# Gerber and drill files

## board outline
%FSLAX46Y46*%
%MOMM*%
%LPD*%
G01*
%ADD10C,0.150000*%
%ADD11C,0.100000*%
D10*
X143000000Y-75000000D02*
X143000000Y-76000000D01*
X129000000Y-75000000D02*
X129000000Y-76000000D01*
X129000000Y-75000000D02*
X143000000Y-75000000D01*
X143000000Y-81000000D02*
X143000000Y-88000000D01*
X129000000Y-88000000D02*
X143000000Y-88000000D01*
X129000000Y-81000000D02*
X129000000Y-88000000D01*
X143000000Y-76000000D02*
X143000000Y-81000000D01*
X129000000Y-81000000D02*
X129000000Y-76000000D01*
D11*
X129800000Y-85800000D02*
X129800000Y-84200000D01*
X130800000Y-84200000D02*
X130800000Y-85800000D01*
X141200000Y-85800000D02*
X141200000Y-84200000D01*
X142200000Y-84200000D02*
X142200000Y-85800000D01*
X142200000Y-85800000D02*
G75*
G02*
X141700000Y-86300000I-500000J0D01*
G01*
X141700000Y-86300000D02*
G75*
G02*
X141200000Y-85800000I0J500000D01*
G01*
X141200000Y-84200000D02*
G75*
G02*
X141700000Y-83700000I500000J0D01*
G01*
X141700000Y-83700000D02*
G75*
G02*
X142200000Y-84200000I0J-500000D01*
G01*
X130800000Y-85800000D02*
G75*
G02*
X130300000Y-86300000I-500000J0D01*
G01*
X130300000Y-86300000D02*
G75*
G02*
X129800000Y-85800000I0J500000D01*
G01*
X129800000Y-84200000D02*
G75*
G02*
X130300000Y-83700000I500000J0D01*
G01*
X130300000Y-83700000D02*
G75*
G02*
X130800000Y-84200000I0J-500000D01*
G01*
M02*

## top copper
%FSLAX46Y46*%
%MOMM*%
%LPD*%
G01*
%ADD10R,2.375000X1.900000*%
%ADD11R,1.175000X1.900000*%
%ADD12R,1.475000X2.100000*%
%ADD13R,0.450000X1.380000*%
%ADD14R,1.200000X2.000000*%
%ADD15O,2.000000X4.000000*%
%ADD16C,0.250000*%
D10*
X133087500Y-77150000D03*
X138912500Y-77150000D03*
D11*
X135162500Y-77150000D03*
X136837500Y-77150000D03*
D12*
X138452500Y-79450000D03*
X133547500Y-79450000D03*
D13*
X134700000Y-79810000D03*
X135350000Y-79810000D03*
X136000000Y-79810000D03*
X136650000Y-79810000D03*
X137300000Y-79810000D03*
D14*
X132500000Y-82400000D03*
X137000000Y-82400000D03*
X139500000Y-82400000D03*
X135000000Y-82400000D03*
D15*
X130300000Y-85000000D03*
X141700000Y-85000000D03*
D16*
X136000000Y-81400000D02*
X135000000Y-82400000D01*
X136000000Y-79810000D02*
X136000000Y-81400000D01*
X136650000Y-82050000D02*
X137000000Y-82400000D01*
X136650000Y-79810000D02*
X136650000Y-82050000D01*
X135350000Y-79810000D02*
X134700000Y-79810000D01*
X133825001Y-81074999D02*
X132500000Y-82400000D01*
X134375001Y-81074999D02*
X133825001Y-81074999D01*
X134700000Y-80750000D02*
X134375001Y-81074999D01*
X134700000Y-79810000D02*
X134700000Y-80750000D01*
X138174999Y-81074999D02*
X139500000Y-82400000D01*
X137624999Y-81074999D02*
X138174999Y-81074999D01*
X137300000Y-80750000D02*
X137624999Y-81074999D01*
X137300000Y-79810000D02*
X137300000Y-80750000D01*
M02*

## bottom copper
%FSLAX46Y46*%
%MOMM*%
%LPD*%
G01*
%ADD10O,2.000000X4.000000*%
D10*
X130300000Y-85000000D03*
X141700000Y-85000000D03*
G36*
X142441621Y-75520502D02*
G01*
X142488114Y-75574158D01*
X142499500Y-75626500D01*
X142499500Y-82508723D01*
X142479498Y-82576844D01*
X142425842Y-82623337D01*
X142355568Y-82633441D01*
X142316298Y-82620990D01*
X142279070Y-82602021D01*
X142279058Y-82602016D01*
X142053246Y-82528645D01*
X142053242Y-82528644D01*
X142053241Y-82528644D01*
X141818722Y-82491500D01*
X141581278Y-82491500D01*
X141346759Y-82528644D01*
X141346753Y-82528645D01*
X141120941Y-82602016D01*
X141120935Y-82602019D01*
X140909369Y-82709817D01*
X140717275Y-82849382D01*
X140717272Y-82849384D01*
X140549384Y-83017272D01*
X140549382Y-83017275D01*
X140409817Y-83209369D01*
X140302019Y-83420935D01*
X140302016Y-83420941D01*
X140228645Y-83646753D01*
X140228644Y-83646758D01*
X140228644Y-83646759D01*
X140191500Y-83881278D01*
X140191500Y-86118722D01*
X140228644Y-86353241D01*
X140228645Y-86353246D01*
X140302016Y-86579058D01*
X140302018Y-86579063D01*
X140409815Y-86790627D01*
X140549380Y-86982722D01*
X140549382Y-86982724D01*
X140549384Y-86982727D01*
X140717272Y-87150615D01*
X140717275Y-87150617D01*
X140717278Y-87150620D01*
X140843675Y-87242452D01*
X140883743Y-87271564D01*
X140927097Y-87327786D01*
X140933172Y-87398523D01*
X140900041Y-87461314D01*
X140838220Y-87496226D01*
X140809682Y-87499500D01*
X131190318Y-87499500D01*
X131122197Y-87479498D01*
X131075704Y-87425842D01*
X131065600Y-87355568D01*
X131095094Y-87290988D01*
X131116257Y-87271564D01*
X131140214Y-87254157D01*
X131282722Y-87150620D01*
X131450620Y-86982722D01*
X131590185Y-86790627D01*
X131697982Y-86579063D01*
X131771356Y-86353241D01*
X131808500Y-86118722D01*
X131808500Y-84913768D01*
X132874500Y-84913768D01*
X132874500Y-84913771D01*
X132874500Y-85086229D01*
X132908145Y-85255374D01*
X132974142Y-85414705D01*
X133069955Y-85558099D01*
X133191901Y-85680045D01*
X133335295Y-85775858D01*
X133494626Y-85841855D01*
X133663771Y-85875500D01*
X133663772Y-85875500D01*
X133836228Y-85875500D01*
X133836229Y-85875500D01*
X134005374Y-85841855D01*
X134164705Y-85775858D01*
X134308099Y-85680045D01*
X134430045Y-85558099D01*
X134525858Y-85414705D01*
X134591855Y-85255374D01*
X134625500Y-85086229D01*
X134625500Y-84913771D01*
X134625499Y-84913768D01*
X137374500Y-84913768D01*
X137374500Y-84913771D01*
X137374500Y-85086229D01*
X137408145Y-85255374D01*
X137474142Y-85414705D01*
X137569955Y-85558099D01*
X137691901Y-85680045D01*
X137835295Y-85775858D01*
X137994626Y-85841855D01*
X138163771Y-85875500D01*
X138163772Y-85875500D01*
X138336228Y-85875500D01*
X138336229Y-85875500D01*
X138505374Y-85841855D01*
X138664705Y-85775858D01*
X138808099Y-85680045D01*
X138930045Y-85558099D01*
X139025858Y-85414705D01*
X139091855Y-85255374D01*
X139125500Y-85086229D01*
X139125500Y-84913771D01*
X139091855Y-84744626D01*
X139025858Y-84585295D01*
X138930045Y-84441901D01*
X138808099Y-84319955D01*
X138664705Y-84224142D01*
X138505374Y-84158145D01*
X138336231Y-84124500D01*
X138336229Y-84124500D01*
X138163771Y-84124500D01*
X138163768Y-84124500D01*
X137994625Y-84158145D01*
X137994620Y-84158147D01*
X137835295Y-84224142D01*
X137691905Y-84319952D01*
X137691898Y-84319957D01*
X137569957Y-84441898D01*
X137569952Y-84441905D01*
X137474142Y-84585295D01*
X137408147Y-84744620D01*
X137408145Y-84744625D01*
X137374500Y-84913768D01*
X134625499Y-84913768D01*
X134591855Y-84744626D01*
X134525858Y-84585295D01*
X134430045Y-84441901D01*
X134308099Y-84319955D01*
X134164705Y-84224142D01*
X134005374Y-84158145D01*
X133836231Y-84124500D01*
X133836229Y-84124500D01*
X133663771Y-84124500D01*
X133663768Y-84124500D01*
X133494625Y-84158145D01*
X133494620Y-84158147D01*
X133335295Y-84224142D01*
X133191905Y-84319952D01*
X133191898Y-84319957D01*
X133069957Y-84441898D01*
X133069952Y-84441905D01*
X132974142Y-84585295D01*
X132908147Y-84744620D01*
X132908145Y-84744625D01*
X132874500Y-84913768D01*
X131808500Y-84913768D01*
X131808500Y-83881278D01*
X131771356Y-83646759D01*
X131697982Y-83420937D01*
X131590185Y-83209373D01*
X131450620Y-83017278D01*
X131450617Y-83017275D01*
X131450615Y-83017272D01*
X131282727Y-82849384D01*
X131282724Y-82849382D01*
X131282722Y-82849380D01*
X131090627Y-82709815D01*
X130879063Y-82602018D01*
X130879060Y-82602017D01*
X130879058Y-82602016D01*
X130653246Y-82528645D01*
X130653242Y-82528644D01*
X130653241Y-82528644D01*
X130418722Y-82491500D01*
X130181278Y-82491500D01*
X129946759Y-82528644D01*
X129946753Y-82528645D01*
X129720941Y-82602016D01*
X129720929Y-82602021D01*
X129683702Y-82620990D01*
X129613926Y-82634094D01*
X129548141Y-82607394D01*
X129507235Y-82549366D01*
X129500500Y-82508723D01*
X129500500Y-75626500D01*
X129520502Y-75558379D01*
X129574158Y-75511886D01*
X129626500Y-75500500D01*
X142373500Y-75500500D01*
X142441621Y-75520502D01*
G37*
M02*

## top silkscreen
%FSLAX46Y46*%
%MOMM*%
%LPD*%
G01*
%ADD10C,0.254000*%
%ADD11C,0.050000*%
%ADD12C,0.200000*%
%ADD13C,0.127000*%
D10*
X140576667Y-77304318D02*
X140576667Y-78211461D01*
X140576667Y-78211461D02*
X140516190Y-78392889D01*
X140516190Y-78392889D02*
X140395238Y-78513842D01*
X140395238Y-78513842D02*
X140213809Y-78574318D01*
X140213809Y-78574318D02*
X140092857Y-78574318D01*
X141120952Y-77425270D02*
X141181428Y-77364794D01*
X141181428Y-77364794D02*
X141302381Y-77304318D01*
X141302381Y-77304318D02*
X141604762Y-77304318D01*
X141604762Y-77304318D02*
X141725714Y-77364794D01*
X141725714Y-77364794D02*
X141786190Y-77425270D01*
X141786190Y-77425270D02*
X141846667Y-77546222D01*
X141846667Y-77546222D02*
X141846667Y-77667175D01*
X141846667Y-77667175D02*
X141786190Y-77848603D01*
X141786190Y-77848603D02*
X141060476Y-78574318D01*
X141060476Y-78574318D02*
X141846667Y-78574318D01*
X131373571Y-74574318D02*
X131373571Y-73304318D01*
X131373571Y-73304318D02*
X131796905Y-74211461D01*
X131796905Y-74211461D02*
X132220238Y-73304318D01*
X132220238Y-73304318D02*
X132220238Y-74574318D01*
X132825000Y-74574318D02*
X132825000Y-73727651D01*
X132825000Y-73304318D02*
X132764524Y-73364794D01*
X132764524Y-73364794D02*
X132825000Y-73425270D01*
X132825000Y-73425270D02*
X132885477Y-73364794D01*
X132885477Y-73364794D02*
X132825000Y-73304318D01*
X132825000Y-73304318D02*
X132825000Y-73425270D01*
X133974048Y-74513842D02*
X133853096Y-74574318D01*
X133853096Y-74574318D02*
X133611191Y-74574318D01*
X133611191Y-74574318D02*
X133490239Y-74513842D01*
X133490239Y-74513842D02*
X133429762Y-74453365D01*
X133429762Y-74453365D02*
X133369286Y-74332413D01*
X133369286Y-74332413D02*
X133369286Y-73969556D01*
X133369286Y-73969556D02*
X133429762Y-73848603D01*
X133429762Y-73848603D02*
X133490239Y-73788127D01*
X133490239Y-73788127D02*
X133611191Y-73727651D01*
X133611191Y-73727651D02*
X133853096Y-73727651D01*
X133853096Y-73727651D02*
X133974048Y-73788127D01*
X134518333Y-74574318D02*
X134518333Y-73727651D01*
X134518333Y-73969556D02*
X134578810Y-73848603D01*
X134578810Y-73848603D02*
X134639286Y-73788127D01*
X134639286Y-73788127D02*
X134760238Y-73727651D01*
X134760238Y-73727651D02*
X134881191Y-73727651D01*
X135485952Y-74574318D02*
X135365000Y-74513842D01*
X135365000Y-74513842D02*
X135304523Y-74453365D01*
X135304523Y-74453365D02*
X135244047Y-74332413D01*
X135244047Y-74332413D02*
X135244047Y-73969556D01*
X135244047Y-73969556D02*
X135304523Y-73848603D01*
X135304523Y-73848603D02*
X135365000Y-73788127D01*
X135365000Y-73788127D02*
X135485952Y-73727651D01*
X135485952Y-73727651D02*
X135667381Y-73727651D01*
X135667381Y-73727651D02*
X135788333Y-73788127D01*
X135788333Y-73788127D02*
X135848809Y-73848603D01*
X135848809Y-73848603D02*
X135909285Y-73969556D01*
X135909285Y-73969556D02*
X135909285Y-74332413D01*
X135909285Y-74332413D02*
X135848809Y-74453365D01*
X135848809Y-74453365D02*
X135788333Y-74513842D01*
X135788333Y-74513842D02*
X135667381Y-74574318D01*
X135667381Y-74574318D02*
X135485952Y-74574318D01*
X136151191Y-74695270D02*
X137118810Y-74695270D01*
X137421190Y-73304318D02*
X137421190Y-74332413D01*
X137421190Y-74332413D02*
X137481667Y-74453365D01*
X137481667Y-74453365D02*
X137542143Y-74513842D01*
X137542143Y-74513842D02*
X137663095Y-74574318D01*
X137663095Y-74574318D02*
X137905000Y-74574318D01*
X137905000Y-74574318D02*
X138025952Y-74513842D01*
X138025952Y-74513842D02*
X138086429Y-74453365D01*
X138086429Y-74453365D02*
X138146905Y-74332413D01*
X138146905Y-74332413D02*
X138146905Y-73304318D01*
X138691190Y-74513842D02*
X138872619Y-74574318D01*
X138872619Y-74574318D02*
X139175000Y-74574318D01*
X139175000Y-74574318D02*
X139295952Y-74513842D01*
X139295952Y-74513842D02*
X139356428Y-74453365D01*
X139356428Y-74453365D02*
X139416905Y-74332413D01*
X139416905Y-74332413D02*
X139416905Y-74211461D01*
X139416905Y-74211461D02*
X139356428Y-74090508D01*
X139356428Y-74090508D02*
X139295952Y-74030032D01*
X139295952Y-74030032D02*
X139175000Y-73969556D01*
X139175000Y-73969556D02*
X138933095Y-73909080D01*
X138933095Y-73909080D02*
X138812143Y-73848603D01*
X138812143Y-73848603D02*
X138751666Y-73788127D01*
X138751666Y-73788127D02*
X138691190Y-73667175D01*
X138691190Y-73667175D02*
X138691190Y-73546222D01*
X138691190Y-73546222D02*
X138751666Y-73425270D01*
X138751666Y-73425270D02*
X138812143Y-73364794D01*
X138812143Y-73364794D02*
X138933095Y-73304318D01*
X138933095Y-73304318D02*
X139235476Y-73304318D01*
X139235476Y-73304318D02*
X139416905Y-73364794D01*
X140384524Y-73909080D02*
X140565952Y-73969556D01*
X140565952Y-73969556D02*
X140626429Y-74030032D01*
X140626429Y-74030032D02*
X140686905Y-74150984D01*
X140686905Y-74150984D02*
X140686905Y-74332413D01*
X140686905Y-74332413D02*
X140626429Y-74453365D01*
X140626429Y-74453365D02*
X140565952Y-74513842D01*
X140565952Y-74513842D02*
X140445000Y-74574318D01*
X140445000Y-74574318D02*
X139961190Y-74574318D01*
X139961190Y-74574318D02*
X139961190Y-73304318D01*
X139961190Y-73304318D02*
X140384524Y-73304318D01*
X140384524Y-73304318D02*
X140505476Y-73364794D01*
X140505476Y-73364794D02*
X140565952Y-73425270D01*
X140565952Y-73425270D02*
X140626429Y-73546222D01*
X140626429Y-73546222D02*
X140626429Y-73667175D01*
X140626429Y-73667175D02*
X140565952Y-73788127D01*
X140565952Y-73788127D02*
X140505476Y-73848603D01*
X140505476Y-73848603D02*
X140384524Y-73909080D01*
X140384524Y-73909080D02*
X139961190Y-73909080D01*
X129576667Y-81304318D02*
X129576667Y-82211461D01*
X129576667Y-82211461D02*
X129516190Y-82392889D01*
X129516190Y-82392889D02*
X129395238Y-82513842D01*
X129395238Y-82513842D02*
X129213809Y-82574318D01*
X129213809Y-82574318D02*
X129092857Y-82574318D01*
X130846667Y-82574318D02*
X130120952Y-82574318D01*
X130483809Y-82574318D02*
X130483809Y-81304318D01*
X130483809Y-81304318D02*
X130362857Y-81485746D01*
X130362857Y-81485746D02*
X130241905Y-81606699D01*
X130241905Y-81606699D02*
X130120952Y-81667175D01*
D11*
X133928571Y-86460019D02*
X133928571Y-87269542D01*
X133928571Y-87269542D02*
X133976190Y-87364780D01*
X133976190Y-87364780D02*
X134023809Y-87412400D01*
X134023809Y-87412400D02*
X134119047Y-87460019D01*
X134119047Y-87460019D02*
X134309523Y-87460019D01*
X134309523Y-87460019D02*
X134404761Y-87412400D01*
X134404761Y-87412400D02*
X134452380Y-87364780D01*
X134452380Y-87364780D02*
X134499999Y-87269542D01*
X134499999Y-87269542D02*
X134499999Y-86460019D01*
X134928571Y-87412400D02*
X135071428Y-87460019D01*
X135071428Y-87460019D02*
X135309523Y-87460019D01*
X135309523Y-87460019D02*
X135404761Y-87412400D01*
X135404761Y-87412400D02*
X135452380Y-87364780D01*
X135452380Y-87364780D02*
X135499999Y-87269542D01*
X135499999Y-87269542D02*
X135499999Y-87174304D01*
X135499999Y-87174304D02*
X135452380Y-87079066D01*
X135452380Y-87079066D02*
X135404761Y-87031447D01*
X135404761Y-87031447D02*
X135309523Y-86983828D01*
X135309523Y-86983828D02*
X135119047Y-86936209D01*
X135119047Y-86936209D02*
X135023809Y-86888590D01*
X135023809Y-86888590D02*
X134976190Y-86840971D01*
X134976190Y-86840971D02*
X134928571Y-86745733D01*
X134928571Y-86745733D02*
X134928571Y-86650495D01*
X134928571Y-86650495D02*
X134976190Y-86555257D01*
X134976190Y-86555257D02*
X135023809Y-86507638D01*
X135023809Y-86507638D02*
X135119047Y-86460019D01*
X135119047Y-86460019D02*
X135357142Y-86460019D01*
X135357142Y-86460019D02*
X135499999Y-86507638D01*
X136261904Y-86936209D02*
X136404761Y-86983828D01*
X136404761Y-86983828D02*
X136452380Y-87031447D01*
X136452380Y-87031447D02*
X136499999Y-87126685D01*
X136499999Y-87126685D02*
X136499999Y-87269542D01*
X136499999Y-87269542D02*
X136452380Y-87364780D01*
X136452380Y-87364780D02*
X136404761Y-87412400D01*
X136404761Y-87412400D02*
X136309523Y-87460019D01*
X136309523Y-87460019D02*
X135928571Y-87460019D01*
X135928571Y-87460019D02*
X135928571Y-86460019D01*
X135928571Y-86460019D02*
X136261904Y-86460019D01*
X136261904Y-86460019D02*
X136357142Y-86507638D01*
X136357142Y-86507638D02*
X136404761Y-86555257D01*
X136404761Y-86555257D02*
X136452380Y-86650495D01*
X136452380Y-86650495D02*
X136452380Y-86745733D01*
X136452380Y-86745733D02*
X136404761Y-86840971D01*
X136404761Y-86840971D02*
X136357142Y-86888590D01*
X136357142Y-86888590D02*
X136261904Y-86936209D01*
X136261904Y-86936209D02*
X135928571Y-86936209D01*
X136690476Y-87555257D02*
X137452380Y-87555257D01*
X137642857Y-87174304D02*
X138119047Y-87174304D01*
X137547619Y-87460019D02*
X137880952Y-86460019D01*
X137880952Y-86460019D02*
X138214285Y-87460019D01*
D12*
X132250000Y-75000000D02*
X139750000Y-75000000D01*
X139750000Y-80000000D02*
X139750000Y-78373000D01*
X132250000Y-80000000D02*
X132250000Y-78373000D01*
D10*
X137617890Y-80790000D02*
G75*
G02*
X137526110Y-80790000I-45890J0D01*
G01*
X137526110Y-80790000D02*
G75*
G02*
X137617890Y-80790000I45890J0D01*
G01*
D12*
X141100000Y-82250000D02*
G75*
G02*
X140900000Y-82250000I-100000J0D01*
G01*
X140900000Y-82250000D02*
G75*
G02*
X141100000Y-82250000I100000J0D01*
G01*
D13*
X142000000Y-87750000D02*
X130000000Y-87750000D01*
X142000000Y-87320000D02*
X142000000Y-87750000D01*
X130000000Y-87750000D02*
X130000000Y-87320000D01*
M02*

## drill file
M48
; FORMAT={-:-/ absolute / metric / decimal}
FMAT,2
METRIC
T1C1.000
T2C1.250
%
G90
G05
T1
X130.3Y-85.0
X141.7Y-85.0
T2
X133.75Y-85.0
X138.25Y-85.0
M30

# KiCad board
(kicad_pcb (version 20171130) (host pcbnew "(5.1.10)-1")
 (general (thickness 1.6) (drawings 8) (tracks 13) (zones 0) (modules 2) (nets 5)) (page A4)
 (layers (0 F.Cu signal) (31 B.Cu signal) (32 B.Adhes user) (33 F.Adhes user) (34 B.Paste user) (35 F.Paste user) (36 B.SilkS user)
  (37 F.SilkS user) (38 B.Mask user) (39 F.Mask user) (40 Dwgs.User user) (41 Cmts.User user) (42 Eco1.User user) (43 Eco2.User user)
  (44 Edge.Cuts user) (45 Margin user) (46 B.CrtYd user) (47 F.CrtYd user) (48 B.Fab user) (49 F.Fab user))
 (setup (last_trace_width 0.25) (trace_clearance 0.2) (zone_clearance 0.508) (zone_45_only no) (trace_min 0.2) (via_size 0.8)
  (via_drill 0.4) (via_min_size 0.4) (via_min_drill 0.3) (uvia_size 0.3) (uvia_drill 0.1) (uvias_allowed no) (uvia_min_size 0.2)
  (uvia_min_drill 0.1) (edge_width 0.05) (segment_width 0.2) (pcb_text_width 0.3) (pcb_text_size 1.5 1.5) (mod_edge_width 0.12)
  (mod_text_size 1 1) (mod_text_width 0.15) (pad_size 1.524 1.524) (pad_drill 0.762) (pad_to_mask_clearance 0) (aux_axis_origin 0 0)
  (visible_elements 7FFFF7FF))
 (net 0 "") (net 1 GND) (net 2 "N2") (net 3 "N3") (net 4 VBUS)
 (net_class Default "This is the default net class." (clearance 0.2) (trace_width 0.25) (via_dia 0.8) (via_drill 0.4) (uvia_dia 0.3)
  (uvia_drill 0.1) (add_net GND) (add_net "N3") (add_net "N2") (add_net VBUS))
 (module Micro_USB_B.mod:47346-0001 (layer F.Cu) (at 136 75)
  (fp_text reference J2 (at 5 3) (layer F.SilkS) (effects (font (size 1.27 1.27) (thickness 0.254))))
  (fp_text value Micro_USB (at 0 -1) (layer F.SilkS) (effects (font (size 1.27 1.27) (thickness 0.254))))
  (fp_line (start -3.75 0) (end 3.75 0) (layer F.SilkS) (width 0.2))
  (fp_line (start 3.75 5) (end 3.75 3.373) (layer F.SilkS) (width 0.2))
  (fp_line (start -3.75 5) (end -3.75 3.373) (layer F.SilkS) (width 0.2))
  (fp_circle (center 1.572 5.79) (end 1.52611 5.79) (layer F.SilkS) (width 0.254))
  (pad 11 smd rect (at -2.9125 2.15 90) (size 1.9 2.375) (layers F.Cu F.Paste F.Mask))
  (pad 10 smd rect (at 2.9125 2.15 90) (size 1.9 2.375) (layers F.Cu F.Paste F.Mask))
  (pad 9 smd rect (at -0.8375 2.15) (size 1.175 1.9) (layers F.Cu F.Paste F.Mask))
  (pad 8 smd rect (at 0.8375 2.15) (size 1.175 1.9) (layers F.Cu F.Paste F.Mask))
  (pad 7 smd rect (at 2.4525 4.45) (size 1.475 2.1) (layers F.Cu F.Paste F.Mask))
  (pad 6 smd rect (at -2.4525 4.45) (size 1.475 2.1) (layers F.Cu F.Paste F.Mask))
  (pad 5 smd rect (at -1.3 4.81) (size 0.45 1.38) (layers F.Cu F.Paste F.Mask) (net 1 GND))
  (pad 4 smd rect (at -0.65 4.81) (size 0.45 1.38) (layers F.Cu F.Paste F.Mask) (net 1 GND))
  (pad 3 smd rect (at 0 4.81) (size 0.45 1.38) (layers F.Cu F.Paste F.Mask) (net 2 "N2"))
  (pad 2 smd rect (at 0.65 4.81) (size 0.45 1.38) (layers F.Cu F.Paste F.Mask) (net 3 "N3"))
  (pad 1 smd rect (at 1.3 4.81) (size 0.45 1.38) (layers F.Cu F.Paste F.Mask) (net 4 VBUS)))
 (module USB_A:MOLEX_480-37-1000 (layer F.Cu) (at 136 85)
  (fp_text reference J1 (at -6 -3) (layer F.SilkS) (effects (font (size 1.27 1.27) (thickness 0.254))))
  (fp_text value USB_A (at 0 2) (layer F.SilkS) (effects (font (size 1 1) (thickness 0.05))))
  (fp_line (start -6.2 0.8) (end -6.2 -0.8) (layer Edge.Cuts) (width 0.1))
  (fp_line (start -5.2 -0.8) (end -5.2 0.8) (layer Edge.Cuts) (width 0.1))
  (fp_line (start 5.2 0.8) (end 5.2 -0.8) (layer Edge.Cuts) (width 0.1))
  (fp_line (start 6.2 -0.8) (end 6.2 0.8) (layer Edge.Cuts) (width 0.1))
  (fp_circle (center 5 -2.75) (end 5.1 -2.75) (layer F.SilkS) (width 0.2))
  (fp_line (start 6 2.75) (end -6 2.75) (layer F.SilkS) (width 0.127))
  (fp_line (start 6 2.32) (end 6 2.75) (layer F.SilkS) (width 0.127))
  (fp_line (start -6 2.75) (end -6 2.32) (layer F.SilkS) (width 0.127))
  (fp_arc (start 5.7 0.8) (end 5.7 1.3) (angle -90) (layer Edge.Cuts) (width 0.1))
  (fp_arc (start 5.7 0.8) (end 5.2 0.8) (angle -90) (layer Edge.Cuts) (width 0.1))
  (fp_arc (start 5.7 -0.8) (end 5.7 -1.3) (angle -90) (layer Edge.Cuts) (width 0.1))
  (fp_arc (start 5.7 -0.8) (end 6.2 -0.8) (angle -90) (layer Edge.Cuts) (width 0.1))
  (fp_arc (start -5.7 0.8) (end -5.7 1.3) (angle -90) (layer Edge.Cuts) (width 0.1))
  (fp_arc (start -5.7 0.8) (end -6.2 0.8) (angle -90) (layer Edge.Cuts) (width 0.1))
  (fp_arc (start -5.7 -0.8) (end -5.7 -1.3) (angle -90) (layer Edge.Cuts) (width 0.1))
  (fp_arc (start -5.7 -0.8) (end -5.2 -0.8) (angle -90) (layer Edge.Cuts) (width 0.1))
  (pad Hole np_thru_hole circle (at -2.25 0) (size 1.25 1.25) (drill 1.25) (layers *.Cu *.Mask))
  (pad Hole np_thru_hole circle (at 2.25 0) (size 1.25 1.25) (drill 1.25) (layers *.Cu *.Mask))
  (pad 4 smd rect (at -3.5 -2.6) (size 1.2 2) (layers F.Cu F.Paste) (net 1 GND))
  (pad 2 smd rect (at 1 -2.6) (size 1.2 2) (layers F.Cu F.Paste) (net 3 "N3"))
  (pad 1 smd rect (at 3.5 -2.6) (size 1.2 2) (layers F.Cu F.Paste) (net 4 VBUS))
  (pad 3 smd rect (at -1 -2.6) (size 1.2 2) (layers F.Cu F.Paste) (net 2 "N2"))
  (pad S1 thru_hole oval (at -5.7 0 90) (size 4 2) (drill 1) (layers *.Cu *.Mask))
  (pad S2 thru_hole oval (at 5.7 0 90) (size 4 2) (drill 1) (layers *.Cu *.Mask)))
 (gr_line (start 143 75) (end 143 76) (layer Edge.Cuts) (width 0.15))
 (gr_line (start 129 75) (end 129 76) (layer Edge.Cuts) (width 0.15))
 (gr_line (start 129 75) (end 143 75) (layer Edge.Cuts) (width 0.15))
 (gr_line (start 143 81) (end 143 88) (layer Edge.Cuts) (width 0.15))
 (gr_line (start 129 88) (end 143 88) (layer Edge.Cuts) (width 0.15))
 (gr_line (start 129 81) (end 129 88) (layer Edge.Cuts) (width 0.15))
 (gr_line (start 143 76) (end 143 81) (layer Edge.Cuts) (width 0.15))
 (gr_line (start 129 81) (end 129 76) (layer Edge.Cuts) (width 0.15))
 (segment (start 136 81.4) (end 135 82.4) (width 0.25) (layer F.Cu) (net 2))
 (segment (start 136 79.81) (end 136 81.4) (width 0.25) (layer F.Cu) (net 2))
 (segment (start 136.65 82.05) (end 137 82.4) (width 0.25) (layer F.Cu) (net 3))
 (segment (start 136.65 79.81) (end 136.65 82.05) (width 0.25) (layer F.Cu) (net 3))
 (segment (start 135.35 79.81) (end 134.7 79.81) (width 0.25) (layer F.Cu) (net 1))
 (segment (start 133.825001 81.074999) (end 132.5 82.4) (width 0.25) (layer F.Cu) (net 1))
 (segment (start 134.375001 81.074999) (end 133.825001 81.074999) (width 0.25) (layer F.Cu) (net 1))
 (segment (start 134.7 80.75) (end 134.375001 81.074999) (width 0.25) (layer F.Cu) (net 1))
 (segment (start 134.7 79.81) (end 134.7 80.75) (width 0.25) (layer F.Cu) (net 1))
 (segment (start 138.174999 81.074999) (end 139.5 82.4) (width 0.25) (layer F.Cu) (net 4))
 (segment (start 137.624999 81.074999) (end 138.174999 81.074999) (width 0.25) (layer F.Cu) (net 4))
 (segment (start 137.3 80.75) (end 137.624999 81.074999) (width 0.25) (layer F.Cu) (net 4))
 (segment (start 137.3 79.81) (end 137.3 80.75) (width 0.25) (layer F.Cu) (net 4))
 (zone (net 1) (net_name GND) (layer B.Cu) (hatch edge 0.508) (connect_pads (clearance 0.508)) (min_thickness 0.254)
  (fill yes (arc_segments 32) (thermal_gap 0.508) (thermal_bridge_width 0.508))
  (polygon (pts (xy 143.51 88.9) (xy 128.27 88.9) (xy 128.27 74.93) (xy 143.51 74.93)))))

